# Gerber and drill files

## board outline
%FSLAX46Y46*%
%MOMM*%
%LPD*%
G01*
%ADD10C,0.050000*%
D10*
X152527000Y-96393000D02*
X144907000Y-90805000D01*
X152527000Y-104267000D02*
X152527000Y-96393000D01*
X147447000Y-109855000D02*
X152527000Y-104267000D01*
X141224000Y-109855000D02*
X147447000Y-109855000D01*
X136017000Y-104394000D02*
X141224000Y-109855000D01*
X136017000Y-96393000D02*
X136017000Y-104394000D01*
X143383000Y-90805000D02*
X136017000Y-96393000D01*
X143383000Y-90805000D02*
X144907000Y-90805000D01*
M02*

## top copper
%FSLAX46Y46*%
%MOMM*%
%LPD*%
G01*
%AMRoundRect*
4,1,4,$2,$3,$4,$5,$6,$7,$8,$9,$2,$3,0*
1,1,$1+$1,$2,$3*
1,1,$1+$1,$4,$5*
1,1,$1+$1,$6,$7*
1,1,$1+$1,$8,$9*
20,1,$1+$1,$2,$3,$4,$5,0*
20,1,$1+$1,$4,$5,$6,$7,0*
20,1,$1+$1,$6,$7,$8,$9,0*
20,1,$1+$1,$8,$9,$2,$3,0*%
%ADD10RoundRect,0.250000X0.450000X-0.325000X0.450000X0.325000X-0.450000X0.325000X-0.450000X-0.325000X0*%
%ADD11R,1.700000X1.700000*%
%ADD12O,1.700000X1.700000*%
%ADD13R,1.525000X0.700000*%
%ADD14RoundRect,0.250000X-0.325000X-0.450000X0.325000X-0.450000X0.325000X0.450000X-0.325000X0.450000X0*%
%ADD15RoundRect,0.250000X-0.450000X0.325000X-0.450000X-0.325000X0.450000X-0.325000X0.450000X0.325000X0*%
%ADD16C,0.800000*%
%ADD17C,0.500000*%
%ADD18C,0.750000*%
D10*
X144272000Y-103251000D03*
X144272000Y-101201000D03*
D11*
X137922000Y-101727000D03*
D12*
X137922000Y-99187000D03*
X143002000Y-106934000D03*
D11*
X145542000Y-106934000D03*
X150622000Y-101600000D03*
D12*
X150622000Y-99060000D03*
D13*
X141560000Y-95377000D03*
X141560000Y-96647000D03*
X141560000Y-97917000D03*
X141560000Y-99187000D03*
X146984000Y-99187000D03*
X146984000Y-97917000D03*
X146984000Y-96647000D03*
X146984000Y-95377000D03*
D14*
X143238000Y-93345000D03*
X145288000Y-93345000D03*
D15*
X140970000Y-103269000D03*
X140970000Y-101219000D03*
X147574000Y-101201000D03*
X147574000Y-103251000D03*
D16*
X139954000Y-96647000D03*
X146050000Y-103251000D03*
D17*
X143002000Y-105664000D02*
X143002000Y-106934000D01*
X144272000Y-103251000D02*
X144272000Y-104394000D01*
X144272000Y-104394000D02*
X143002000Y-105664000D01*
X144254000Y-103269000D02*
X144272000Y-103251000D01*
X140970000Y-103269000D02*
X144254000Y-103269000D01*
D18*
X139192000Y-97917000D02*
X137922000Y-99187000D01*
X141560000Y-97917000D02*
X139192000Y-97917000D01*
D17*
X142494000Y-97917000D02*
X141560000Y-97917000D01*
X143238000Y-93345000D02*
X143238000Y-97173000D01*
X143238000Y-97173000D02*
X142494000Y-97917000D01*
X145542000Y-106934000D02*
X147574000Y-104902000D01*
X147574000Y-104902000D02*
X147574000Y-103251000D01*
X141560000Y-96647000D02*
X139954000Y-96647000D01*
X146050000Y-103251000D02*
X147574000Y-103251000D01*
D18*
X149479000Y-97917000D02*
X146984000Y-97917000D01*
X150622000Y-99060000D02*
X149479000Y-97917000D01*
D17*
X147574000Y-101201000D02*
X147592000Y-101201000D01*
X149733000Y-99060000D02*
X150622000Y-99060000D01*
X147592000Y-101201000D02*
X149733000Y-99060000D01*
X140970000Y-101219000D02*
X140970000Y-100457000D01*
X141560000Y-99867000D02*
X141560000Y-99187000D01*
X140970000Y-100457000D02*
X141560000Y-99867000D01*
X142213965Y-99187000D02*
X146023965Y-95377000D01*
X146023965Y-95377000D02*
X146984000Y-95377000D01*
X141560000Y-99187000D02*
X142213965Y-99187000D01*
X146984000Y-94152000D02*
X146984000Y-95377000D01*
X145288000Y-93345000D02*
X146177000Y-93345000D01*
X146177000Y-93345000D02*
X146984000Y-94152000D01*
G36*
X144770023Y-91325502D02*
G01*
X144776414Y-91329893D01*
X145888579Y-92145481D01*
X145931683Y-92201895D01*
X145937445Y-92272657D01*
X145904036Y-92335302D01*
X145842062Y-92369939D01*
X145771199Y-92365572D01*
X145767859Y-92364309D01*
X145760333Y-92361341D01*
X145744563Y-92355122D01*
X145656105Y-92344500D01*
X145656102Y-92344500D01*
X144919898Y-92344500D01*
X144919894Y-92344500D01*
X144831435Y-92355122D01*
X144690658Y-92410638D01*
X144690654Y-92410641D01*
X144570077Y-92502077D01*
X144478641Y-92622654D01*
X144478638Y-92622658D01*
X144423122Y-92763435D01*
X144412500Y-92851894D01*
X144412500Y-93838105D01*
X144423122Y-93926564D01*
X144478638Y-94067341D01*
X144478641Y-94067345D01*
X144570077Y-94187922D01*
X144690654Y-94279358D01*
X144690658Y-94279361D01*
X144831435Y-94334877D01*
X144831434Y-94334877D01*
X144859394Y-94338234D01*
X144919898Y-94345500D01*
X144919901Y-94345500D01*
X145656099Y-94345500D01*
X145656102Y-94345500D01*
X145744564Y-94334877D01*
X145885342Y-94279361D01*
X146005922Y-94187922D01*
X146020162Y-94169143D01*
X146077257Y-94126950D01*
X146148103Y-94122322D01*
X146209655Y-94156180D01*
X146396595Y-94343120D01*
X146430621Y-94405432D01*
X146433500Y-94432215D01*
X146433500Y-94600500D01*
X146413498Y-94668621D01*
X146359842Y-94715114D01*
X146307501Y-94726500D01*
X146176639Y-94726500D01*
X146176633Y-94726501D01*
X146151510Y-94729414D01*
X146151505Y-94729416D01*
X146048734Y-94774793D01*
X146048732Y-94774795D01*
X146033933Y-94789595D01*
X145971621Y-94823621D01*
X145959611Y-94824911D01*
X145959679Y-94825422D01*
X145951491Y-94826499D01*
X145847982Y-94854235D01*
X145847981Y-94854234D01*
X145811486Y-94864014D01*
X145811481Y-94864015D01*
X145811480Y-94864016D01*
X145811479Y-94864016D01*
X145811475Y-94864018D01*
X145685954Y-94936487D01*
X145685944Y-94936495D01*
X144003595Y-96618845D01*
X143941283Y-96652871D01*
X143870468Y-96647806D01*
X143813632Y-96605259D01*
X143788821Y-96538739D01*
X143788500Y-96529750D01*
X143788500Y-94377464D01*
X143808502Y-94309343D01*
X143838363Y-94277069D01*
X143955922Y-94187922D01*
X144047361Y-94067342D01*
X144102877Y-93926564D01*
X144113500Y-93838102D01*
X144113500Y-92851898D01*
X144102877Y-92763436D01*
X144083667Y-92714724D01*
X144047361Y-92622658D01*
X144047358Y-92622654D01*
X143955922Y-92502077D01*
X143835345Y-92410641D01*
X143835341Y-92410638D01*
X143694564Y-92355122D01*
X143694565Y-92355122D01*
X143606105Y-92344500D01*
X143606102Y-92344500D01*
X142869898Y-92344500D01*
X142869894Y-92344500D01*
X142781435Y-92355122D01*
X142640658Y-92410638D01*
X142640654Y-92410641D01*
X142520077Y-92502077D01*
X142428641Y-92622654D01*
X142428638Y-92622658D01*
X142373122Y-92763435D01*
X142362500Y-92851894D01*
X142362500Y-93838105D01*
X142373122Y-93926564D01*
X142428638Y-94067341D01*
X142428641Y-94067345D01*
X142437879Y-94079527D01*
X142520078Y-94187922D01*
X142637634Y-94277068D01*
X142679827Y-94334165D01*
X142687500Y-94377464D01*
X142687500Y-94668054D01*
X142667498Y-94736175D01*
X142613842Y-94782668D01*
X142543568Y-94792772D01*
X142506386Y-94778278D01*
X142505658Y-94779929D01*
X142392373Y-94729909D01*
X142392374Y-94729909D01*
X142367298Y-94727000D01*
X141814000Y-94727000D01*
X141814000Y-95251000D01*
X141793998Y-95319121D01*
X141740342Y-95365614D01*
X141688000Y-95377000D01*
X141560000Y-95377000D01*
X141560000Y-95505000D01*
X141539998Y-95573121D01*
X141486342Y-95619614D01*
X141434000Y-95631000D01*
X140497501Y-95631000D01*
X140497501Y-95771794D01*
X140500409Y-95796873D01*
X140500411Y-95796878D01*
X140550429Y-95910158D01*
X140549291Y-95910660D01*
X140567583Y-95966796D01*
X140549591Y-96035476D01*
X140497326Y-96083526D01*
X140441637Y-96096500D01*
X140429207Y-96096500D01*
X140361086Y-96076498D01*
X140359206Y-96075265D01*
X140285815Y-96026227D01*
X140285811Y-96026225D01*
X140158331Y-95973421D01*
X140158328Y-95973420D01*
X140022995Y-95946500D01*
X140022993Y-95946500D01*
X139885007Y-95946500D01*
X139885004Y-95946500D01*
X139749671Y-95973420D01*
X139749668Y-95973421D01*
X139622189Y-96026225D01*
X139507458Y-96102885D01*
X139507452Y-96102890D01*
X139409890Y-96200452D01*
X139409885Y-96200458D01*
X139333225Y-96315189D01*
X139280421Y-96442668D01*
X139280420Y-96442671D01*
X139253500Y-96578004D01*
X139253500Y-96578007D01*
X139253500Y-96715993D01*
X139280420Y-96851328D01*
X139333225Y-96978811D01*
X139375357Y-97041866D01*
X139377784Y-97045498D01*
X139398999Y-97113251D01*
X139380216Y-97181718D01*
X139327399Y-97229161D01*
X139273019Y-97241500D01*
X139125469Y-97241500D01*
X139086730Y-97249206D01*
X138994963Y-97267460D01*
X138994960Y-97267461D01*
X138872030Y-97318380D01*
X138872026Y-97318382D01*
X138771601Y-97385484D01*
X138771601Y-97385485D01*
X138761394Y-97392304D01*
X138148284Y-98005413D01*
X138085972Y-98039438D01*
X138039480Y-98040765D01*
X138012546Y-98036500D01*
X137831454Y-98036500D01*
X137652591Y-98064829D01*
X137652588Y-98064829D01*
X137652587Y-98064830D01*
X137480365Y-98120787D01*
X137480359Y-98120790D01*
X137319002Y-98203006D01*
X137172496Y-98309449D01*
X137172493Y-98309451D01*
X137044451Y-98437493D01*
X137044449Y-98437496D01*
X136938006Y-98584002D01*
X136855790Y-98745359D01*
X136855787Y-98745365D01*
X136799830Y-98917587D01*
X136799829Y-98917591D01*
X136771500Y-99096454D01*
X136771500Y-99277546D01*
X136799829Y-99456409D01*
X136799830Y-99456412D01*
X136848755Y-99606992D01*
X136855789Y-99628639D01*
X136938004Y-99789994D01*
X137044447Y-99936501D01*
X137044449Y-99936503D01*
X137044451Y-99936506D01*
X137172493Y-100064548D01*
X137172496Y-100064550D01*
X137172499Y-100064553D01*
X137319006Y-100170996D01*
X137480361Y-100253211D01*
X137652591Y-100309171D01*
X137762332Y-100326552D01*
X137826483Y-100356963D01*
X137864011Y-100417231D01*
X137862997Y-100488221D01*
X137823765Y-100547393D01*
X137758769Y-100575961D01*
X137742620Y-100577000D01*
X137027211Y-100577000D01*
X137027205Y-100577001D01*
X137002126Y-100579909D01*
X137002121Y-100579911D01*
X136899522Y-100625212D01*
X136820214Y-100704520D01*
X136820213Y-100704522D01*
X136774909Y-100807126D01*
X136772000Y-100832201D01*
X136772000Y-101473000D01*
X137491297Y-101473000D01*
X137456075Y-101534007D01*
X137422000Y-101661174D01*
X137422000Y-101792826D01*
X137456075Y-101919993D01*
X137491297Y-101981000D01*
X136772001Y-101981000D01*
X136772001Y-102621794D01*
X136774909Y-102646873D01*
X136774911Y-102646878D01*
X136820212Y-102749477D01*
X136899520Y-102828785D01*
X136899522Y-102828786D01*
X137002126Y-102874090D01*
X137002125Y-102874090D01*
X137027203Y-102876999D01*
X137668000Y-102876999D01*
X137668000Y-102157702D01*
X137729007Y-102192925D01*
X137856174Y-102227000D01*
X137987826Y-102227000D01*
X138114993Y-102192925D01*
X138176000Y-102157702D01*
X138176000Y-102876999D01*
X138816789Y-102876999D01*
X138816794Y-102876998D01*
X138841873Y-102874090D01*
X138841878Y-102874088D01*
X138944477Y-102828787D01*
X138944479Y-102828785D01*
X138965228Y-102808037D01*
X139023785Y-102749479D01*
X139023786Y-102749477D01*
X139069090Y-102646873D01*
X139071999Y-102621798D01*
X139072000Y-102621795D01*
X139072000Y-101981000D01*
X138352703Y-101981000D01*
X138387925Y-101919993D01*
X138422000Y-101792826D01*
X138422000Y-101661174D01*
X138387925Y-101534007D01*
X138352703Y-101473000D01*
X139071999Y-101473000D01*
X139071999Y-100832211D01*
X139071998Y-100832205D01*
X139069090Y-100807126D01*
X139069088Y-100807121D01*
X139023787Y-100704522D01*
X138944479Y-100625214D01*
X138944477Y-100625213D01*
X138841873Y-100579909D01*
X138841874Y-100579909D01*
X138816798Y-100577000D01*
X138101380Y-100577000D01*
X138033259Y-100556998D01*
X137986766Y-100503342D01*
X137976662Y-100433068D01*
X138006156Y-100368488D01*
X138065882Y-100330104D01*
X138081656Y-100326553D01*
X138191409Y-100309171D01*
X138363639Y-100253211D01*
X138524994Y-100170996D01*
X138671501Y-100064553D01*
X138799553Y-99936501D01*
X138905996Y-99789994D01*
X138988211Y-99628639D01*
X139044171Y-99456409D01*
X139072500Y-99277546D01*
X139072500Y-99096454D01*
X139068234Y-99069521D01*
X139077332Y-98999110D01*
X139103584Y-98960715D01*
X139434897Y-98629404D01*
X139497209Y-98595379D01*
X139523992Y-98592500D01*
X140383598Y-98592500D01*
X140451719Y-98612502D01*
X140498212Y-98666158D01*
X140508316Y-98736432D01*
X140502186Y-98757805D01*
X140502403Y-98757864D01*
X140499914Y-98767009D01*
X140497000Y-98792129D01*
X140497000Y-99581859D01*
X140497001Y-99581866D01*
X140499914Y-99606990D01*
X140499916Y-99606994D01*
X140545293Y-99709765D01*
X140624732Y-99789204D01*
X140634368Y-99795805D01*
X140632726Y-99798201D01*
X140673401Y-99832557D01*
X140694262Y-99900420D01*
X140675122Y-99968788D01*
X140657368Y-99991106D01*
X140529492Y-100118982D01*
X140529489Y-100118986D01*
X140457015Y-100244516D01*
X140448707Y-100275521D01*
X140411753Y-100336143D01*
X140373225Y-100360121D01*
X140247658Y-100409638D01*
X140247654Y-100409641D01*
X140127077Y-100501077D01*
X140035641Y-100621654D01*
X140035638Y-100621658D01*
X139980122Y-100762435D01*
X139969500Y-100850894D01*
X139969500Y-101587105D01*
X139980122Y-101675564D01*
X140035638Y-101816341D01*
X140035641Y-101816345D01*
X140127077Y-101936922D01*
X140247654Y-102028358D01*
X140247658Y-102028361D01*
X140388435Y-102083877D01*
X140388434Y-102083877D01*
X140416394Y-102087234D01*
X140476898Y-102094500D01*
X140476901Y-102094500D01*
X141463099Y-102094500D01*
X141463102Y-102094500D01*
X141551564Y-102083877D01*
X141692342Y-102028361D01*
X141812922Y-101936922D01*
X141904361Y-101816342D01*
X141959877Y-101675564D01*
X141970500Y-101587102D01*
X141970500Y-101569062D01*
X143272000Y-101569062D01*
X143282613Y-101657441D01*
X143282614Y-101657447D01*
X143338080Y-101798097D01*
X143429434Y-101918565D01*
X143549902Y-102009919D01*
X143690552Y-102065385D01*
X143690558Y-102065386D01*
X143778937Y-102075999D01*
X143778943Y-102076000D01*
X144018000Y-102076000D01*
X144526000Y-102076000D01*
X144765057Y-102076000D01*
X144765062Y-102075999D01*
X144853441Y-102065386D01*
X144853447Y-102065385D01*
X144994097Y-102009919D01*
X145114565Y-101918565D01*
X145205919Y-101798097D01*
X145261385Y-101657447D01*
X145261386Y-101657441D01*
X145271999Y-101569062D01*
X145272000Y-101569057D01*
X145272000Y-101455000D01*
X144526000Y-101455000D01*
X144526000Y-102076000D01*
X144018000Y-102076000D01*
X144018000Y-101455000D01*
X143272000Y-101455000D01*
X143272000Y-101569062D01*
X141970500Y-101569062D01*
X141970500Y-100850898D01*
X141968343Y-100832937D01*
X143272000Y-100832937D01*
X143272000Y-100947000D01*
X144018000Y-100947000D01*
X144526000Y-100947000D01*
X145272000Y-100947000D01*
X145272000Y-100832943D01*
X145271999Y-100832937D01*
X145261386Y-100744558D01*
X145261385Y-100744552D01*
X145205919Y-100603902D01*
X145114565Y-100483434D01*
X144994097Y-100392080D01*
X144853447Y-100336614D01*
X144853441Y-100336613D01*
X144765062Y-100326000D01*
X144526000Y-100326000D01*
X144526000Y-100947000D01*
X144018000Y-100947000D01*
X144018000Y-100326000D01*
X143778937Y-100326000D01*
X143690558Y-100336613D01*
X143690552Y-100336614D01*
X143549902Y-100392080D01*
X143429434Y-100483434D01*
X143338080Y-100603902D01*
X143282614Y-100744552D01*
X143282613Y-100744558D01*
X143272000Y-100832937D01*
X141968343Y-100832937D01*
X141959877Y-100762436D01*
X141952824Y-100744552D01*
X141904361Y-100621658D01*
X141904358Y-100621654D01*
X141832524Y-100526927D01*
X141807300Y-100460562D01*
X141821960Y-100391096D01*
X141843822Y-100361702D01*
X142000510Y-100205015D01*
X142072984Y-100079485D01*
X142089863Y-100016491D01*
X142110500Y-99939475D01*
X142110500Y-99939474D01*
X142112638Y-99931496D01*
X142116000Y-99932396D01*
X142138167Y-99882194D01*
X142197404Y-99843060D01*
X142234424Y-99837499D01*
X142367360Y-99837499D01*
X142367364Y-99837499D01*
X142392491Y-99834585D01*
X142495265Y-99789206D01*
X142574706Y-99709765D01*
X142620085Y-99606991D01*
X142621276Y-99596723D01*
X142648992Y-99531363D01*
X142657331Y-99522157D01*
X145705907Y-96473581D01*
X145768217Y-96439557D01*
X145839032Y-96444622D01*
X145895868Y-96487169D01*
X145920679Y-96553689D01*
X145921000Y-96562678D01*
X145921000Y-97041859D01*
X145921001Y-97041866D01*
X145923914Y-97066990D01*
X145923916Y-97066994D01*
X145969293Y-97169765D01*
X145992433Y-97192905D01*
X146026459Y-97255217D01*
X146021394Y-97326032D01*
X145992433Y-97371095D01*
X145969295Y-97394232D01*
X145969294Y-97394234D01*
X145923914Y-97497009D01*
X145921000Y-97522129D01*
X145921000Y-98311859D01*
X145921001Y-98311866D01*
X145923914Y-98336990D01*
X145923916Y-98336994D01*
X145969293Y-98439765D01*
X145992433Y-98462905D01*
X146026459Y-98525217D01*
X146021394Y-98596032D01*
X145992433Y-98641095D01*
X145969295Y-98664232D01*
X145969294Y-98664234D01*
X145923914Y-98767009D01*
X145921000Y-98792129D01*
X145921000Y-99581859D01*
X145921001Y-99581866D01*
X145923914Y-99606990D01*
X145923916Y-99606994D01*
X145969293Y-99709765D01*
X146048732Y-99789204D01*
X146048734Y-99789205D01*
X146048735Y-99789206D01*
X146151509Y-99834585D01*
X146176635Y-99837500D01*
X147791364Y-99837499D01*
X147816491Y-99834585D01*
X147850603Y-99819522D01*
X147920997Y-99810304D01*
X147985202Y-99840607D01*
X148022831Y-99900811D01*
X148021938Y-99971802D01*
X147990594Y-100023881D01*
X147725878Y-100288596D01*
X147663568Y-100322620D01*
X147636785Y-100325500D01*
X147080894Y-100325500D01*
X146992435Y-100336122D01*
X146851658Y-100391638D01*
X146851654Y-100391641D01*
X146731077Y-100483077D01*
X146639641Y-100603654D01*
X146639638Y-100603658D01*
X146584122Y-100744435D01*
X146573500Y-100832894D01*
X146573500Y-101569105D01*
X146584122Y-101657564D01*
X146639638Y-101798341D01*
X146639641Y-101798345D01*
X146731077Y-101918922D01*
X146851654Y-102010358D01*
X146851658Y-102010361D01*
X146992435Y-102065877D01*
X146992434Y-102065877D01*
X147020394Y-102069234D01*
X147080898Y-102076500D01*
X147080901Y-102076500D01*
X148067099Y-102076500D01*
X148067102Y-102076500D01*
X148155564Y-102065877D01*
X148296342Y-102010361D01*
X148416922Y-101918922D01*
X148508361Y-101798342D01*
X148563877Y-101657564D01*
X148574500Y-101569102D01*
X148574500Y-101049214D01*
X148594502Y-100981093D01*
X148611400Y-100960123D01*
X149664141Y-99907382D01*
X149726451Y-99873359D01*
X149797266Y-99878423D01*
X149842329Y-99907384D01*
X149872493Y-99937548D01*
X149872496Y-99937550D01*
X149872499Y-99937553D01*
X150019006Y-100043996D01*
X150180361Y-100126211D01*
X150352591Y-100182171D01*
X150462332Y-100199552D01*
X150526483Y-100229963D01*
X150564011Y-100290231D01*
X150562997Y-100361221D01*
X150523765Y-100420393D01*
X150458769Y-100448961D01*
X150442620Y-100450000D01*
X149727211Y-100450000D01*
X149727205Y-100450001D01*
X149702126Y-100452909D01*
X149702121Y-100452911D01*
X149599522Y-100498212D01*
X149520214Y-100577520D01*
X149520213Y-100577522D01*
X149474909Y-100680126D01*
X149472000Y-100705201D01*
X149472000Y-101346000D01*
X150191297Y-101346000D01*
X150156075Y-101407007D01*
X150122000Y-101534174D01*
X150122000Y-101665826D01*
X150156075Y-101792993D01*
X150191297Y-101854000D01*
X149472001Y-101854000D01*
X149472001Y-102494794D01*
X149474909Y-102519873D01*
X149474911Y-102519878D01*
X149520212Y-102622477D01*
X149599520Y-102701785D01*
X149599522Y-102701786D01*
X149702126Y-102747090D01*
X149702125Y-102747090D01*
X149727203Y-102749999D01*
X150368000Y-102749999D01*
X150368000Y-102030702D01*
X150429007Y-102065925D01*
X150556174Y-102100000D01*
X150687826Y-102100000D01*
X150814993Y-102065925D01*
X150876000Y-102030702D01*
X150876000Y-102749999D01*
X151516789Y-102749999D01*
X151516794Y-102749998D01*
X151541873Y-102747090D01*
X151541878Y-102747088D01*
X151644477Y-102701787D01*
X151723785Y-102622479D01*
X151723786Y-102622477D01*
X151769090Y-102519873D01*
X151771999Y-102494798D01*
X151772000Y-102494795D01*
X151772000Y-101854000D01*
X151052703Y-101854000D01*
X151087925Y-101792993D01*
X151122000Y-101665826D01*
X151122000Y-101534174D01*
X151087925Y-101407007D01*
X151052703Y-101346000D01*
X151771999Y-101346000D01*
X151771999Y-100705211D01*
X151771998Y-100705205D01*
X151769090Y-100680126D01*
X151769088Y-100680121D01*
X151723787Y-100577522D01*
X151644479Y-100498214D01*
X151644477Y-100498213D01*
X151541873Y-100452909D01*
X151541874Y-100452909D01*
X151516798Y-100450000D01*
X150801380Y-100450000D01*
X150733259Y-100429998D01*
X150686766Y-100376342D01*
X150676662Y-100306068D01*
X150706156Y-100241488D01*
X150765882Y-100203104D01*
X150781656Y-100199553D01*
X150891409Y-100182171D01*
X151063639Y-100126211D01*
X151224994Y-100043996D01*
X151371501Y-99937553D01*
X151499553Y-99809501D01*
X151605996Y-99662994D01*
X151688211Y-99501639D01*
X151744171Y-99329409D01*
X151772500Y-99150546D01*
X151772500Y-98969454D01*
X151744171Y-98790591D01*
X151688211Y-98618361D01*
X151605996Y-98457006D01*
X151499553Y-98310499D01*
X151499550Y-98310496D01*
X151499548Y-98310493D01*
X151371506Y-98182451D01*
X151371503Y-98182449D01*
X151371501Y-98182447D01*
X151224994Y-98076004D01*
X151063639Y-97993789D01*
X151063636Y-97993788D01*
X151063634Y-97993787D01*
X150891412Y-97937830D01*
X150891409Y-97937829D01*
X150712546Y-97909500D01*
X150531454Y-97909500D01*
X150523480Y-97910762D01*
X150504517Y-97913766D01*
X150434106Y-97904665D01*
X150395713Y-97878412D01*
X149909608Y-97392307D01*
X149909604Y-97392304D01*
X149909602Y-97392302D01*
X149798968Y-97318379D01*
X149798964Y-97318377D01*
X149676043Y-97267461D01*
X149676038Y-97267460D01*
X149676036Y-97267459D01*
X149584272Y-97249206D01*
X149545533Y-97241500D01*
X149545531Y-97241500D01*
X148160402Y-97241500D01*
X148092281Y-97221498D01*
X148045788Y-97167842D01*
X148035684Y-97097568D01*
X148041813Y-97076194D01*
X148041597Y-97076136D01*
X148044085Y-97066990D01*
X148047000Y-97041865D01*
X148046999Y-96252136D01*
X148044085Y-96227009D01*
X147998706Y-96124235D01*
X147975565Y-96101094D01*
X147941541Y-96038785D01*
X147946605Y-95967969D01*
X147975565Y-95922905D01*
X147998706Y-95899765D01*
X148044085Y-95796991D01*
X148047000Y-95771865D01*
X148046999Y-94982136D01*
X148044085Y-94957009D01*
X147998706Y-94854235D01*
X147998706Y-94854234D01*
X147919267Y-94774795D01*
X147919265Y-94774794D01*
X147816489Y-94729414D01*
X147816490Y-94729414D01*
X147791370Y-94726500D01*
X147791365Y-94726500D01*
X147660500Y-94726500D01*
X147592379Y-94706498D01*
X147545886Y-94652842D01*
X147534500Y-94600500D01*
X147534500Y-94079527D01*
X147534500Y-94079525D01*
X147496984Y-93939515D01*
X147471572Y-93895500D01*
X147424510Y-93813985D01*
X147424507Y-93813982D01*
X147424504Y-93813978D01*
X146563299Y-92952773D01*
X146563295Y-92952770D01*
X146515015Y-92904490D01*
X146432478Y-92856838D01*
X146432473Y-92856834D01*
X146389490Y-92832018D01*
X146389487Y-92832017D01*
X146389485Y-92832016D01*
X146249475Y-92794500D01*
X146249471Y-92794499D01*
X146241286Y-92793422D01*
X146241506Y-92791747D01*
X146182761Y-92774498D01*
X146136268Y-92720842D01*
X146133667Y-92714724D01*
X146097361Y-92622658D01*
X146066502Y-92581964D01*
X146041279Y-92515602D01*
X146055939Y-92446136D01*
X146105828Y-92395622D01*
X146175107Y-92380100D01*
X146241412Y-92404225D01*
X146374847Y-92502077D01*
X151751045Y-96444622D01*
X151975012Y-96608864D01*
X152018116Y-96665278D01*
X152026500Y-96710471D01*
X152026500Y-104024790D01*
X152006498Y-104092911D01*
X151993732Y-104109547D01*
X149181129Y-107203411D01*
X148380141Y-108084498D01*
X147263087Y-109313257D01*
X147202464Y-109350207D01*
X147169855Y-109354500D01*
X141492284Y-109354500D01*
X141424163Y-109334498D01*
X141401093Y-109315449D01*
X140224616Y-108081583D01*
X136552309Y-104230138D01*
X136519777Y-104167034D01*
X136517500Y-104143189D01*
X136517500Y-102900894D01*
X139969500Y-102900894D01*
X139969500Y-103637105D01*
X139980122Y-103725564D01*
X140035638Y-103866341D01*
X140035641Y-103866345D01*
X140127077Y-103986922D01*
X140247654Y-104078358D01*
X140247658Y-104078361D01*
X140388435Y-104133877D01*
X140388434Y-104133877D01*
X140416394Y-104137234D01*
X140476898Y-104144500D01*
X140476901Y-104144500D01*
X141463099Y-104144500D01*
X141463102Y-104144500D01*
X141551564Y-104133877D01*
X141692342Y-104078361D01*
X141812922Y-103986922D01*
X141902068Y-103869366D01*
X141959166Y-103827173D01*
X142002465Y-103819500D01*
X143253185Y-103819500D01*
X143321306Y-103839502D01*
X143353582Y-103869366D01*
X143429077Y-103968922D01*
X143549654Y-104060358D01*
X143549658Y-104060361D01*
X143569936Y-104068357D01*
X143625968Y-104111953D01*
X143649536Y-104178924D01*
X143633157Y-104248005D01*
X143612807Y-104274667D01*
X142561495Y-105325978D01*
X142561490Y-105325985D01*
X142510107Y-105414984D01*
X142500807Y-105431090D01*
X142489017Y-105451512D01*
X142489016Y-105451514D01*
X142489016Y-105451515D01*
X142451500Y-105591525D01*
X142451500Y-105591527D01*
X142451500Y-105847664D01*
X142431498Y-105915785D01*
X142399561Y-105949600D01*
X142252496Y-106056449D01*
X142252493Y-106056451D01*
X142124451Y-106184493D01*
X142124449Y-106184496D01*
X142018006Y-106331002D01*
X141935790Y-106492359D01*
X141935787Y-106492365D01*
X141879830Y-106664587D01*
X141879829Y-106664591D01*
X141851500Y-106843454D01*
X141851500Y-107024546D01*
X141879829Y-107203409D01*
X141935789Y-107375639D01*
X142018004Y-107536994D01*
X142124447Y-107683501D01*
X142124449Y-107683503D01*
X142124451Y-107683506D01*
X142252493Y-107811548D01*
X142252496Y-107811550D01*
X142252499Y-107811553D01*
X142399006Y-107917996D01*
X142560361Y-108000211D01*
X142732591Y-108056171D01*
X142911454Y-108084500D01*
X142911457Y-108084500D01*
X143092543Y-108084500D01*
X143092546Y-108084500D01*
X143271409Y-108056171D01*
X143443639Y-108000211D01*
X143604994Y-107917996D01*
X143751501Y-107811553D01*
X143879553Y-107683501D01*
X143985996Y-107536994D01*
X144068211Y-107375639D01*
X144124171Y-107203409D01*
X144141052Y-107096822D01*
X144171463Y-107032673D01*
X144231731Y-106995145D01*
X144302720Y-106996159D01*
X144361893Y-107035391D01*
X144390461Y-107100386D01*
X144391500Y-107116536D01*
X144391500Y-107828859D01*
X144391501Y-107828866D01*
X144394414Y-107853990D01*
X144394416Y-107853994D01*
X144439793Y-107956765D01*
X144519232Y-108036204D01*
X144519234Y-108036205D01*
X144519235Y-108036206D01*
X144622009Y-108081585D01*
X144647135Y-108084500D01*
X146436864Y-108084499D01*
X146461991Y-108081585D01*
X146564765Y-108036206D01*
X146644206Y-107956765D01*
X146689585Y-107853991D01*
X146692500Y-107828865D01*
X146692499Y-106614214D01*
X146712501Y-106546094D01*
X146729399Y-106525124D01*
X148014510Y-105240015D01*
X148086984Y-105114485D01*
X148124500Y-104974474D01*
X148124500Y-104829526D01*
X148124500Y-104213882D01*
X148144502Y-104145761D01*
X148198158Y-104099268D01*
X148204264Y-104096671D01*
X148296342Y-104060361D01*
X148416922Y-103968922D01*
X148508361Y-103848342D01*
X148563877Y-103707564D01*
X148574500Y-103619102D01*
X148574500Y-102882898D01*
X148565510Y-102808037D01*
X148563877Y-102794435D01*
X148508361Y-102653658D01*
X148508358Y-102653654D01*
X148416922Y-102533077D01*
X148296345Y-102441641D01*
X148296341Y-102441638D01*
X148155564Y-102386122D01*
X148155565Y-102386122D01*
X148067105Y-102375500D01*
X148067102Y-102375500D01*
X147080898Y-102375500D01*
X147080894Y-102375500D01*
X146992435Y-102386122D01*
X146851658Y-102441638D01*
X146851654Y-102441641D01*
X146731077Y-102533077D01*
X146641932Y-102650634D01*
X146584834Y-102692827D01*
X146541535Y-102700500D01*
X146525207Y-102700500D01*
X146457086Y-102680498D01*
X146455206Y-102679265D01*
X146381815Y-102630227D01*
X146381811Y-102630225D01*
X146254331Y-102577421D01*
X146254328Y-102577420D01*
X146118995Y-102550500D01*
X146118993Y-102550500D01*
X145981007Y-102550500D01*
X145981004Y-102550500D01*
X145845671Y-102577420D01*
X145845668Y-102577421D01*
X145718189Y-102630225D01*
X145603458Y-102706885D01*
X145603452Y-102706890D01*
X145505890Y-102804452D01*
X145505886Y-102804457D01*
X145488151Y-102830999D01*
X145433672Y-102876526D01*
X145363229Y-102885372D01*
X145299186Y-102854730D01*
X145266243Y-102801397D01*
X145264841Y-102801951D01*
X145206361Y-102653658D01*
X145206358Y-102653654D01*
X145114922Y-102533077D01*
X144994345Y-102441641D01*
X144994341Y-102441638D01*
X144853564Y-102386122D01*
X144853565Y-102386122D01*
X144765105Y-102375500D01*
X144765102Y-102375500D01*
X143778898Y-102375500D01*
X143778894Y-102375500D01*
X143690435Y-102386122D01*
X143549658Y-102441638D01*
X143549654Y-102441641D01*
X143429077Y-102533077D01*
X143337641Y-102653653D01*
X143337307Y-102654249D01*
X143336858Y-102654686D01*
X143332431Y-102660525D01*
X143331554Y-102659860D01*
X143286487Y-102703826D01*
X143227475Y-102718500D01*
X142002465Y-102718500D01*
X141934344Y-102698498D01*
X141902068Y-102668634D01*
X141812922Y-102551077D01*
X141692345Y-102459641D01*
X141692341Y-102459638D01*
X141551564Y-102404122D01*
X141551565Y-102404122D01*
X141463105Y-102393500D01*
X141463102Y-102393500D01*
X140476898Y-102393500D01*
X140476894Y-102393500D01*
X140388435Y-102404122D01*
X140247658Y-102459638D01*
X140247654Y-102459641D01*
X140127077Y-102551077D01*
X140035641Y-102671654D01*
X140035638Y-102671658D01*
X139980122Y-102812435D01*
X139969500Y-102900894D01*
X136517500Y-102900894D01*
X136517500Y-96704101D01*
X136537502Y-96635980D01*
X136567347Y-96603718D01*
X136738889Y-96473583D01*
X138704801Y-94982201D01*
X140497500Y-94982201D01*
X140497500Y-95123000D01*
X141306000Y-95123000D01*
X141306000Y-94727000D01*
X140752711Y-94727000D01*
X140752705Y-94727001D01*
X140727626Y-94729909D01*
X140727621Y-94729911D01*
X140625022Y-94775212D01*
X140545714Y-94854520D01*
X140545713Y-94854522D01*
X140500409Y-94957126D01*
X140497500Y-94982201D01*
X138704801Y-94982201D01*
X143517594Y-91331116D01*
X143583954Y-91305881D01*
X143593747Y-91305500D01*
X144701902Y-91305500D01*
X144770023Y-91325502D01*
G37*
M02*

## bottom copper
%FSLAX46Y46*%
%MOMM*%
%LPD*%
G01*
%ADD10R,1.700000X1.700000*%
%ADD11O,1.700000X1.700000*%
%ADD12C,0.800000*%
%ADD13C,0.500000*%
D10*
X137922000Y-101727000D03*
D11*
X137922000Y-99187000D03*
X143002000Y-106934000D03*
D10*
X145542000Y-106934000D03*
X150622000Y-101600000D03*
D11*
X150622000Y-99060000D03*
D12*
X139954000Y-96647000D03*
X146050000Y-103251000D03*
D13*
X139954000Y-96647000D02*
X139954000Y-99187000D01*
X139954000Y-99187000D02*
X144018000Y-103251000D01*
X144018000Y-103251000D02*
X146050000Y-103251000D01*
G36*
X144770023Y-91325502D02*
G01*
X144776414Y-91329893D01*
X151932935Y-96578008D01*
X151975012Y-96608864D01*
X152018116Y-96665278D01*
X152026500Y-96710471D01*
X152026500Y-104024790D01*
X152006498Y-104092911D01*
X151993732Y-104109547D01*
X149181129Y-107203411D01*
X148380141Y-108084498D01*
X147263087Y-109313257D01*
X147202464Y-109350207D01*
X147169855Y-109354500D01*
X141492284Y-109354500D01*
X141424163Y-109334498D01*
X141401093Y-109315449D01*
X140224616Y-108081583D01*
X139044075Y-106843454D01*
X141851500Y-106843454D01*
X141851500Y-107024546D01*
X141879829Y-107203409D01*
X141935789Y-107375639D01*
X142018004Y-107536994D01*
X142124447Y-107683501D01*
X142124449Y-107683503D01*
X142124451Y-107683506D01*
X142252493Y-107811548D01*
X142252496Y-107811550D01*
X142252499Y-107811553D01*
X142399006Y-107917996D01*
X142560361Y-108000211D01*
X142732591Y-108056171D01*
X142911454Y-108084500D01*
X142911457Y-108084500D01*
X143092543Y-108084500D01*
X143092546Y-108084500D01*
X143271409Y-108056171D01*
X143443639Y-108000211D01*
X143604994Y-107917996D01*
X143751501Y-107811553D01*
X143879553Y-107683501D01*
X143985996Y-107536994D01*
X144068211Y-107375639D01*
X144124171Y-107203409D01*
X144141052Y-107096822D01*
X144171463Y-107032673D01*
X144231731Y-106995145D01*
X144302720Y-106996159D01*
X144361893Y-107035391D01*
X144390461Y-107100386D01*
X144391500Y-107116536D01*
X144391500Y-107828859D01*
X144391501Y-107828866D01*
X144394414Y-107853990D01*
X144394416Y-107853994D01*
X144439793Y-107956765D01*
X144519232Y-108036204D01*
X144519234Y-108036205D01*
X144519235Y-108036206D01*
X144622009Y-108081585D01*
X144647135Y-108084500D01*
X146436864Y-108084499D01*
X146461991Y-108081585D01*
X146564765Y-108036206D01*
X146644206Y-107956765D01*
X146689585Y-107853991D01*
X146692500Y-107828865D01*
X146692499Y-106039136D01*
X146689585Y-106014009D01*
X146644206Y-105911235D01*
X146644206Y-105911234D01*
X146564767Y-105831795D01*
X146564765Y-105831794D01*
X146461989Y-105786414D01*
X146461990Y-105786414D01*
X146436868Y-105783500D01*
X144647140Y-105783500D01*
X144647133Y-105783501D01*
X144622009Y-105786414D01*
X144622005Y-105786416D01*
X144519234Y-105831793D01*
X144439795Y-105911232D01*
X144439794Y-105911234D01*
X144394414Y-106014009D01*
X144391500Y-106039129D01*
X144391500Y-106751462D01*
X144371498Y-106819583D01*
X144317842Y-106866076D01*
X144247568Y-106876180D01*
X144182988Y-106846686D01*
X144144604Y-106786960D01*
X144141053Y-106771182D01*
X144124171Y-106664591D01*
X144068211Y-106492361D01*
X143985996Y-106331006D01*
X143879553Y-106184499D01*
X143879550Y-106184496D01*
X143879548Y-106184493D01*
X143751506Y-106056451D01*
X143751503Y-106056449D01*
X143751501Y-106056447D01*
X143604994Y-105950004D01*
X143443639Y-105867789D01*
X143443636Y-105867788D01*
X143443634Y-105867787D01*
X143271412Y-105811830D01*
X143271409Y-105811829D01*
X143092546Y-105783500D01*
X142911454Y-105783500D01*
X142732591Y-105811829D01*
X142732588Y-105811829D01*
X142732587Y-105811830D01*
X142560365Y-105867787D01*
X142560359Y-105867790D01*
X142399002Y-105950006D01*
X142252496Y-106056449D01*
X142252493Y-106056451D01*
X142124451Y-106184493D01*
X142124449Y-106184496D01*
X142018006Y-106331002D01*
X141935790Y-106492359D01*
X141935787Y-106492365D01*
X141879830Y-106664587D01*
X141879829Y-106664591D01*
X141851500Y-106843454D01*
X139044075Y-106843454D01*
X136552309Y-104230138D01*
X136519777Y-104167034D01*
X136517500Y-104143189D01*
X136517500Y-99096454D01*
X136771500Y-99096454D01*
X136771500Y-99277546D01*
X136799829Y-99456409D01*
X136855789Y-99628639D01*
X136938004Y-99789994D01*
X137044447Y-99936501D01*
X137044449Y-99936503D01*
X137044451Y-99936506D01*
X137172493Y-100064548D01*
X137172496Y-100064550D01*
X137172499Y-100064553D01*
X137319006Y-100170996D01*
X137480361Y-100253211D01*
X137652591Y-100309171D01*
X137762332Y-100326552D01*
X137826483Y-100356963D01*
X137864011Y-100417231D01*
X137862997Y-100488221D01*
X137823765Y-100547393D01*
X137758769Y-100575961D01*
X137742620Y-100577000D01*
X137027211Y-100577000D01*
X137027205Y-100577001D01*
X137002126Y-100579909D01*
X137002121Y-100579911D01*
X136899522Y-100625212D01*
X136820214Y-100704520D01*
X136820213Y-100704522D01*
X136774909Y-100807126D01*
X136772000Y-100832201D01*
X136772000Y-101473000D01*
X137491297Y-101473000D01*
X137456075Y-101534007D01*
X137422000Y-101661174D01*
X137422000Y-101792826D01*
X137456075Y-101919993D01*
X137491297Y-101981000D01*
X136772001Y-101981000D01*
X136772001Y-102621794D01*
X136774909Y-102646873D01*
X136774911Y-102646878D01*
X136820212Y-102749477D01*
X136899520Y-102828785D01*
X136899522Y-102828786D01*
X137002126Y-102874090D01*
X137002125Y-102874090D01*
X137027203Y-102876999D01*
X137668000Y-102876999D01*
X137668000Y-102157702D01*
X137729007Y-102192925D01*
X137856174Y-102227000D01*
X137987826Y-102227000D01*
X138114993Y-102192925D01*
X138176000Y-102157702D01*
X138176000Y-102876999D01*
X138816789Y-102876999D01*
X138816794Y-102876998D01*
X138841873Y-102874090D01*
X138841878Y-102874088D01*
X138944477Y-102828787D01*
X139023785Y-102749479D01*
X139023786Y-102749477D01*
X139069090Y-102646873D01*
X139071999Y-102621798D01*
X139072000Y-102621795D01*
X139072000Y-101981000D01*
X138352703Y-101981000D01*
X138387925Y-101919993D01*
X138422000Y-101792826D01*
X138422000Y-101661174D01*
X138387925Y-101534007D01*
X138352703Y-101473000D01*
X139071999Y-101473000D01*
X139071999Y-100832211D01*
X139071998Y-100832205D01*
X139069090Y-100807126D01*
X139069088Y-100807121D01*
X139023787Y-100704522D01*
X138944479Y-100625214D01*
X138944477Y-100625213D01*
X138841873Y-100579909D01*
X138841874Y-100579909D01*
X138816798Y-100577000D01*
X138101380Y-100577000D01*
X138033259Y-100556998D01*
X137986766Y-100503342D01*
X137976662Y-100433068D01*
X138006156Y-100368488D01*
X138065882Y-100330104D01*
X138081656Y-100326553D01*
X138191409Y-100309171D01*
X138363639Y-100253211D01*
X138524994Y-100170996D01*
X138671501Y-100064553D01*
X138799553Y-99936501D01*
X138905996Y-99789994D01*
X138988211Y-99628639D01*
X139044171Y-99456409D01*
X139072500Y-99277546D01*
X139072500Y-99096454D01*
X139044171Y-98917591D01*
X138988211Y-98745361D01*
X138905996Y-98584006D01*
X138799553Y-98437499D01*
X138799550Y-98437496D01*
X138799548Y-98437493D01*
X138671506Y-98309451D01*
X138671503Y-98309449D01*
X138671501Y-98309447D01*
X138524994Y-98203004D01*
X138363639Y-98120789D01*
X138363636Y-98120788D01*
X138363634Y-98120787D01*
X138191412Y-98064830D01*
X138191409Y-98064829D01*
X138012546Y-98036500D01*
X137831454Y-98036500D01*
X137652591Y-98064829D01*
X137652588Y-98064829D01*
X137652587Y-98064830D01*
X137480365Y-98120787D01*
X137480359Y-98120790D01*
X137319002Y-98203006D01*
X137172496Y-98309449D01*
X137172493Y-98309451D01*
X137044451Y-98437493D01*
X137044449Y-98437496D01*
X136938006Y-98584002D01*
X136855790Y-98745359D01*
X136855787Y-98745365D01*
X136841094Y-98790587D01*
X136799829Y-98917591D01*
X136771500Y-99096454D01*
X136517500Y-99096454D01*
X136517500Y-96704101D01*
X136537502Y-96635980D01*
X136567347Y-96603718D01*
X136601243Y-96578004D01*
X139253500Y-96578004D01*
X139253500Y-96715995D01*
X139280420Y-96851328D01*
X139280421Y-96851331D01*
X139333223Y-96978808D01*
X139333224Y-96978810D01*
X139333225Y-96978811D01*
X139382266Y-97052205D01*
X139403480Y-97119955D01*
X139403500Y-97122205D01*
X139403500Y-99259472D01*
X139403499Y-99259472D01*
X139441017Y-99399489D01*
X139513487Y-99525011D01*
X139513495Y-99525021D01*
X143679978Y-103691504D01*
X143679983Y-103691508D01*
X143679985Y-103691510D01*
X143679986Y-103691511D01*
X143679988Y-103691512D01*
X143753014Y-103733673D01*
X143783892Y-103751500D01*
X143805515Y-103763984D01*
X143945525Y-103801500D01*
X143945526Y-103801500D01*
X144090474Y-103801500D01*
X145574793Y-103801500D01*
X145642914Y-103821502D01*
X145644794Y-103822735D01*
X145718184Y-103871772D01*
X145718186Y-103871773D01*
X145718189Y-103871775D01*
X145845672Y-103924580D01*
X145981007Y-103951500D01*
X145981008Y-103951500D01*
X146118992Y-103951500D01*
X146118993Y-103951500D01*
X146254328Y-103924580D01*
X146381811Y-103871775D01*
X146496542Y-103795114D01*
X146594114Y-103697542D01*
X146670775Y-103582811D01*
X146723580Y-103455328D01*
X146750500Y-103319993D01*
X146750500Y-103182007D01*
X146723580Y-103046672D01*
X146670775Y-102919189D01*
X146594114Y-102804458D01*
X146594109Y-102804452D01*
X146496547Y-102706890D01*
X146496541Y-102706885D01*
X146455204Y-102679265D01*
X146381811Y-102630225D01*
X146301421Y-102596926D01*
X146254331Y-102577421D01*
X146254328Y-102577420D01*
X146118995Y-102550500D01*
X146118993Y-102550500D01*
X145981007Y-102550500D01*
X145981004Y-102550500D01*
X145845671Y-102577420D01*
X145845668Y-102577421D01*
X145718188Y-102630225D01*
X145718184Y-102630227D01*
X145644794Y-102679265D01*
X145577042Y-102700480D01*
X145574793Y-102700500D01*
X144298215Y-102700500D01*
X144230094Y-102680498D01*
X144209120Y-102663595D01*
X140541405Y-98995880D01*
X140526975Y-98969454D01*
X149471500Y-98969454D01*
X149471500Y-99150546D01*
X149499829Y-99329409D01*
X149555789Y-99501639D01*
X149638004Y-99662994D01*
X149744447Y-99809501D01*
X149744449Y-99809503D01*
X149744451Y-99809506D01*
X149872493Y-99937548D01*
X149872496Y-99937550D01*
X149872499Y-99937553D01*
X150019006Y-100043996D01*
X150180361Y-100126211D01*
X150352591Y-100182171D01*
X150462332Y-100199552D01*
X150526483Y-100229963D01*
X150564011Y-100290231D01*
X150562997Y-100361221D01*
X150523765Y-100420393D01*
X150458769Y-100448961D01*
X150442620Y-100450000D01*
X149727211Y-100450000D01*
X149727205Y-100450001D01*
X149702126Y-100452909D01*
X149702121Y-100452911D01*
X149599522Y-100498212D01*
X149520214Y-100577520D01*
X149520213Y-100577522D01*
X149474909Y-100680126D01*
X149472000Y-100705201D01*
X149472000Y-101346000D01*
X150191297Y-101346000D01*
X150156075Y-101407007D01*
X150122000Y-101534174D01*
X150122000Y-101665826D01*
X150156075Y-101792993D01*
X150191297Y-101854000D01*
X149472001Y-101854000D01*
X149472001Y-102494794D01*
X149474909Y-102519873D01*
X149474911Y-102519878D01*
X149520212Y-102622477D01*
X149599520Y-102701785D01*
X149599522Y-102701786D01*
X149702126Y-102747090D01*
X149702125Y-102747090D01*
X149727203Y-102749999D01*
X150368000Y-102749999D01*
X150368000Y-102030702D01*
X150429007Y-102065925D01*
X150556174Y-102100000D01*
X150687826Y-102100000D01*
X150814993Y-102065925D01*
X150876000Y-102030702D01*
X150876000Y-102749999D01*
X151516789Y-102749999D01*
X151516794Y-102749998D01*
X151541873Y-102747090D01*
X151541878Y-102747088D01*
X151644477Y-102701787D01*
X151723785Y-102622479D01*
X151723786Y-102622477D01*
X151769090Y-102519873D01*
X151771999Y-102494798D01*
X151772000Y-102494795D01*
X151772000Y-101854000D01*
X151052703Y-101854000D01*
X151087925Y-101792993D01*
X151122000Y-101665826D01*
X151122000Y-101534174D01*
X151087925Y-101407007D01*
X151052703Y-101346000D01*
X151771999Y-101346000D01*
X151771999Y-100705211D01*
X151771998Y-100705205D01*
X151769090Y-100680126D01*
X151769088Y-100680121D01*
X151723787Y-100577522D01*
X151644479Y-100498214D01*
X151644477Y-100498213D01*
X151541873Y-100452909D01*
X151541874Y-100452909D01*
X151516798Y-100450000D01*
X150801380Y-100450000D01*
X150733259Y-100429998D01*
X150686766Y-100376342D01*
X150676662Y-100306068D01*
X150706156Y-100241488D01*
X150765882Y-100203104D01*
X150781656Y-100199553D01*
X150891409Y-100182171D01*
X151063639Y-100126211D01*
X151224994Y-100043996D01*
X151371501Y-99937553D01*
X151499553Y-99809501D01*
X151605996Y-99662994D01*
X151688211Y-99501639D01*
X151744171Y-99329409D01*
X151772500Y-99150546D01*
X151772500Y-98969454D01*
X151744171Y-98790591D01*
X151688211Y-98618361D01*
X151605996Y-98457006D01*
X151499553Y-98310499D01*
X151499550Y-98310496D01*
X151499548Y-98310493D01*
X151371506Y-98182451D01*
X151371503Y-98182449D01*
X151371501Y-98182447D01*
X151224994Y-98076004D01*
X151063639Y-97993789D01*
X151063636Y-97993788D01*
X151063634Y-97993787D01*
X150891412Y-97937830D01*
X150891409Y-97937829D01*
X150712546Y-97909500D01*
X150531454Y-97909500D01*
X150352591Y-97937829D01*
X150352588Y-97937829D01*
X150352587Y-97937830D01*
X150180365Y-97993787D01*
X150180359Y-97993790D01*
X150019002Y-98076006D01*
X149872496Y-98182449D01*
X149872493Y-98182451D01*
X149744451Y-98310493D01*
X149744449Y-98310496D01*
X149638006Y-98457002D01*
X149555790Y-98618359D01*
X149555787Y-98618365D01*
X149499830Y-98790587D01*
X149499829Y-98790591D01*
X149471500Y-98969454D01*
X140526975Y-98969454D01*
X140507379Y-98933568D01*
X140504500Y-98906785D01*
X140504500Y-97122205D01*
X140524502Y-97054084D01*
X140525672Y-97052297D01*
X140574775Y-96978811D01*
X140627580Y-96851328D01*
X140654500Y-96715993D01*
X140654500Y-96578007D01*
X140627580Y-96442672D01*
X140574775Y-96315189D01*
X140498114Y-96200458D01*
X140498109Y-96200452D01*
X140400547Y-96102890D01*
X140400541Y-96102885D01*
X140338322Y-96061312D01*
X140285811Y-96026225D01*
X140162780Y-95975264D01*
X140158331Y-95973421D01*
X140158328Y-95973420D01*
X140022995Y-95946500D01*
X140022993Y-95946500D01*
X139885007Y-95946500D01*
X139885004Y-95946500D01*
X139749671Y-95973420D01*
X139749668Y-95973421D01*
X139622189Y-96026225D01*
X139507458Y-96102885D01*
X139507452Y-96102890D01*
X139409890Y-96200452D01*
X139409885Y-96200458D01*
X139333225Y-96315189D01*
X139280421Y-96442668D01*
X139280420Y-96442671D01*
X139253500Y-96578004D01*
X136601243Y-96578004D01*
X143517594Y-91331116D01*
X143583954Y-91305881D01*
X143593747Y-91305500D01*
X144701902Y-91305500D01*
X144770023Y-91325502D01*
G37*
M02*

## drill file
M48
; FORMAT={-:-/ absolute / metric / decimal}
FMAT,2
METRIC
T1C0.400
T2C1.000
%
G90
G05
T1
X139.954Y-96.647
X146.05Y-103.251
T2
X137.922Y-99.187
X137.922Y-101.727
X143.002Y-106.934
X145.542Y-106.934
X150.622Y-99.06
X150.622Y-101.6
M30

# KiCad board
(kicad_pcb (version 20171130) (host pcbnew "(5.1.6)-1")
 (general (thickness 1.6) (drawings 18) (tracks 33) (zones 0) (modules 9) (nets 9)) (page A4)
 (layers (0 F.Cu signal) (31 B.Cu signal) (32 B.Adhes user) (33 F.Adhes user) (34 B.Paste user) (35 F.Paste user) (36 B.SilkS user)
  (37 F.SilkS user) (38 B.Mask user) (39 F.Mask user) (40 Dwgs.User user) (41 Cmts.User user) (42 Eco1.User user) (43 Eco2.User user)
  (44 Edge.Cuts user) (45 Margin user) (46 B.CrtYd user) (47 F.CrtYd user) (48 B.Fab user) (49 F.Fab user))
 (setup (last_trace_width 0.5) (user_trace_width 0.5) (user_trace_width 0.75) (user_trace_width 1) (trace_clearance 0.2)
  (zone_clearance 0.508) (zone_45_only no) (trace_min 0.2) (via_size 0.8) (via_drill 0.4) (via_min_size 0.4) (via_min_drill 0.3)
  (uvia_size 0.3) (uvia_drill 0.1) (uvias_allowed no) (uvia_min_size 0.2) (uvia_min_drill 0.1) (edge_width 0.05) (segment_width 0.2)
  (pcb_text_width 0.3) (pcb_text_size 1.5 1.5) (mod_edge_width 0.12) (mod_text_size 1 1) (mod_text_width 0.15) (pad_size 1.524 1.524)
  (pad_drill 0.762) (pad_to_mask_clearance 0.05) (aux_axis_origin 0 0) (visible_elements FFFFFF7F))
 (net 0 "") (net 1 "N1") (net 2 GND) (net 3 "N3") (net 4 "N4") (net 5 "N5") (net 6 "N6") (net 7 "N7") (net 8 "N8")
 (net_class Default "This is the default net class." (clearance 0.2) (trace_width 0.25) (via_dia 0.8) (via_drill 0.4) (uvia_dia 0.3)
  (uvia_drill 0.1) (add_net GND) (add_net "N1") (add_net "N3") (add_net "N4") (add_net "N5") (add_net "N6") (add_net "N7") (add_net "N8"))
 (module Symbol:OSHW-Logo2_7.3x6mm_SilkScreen (layer B.Cu) (at 144.145 94.234 180)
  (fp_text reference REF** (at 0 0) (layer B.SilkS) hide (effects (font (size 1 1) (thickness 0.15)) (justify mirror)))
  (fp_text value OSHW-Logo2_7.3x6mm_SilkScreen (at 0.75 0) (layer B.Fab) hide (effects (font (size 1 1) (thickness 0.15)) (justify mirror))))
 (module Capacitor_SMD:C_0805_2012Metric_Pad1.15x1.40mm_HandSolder (layer F.Cu) (at 144.272 102.226 90)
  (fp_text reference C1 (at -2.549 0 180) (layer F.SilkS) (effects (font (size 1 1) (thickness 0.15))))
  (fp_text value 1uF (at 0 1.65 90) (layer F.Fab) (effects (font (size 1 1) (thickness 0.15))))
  (pad 1 smd roundrect (at -1.025 0 90) (size 1.15 1.4) (layers F.Cu F.Paste F.Mask) (roundrect_rratio 0.217391) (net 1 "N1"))
  (pad 2 smd roundrect (at 1.025 0 90) (size 1.15 1.4) (layers F.Cu F.Paste F.Mask) (roundrect_rratio 0.217391) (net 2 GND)))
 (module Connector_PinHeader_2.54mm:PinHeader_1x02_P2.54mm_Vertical (layer F.Cu) (at 137.922 101.727 180)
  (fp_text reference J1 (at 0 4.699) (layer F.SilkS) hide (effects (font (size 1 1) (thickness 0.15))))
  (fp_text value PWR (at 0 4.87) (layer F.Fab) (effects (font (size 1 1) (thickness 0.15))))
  (pad 1 thru_hole rect (at 0 0 180) (size 1.7 1.7) (drill 1) (layers *.Cu *.Mask) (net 2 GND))
  (pad 2 thru_hole oval (at 0 2.54 180) (size 1.7 1.7) (drill 1) (layers *.Cu *.Mask) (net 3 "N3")))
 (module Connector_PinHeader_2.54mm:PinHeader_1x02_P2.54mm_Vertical (layer F.Cu) (at 145.542 106.934 270)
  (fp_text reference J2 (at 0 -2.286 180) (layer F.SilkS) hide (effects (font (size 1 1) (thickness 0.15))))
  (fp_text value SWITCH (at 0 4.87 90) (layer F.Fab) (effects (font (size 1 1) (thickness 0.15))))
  (pad 2 thru_hole oval (at 0 2.54 270) (size 1.7 1.7) (drill 1) (layers *.Cu *.Mask) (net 1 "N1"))
  (pad 1 thru_hole rect (at 0 0 270) (size 1.7 1.7) (drill 1) (layers *.Cu *.Mask) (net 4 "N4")))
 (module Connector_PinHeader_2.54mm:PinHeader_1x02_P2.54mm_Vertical (layer F.Cu) (at 150.622 101.6 180)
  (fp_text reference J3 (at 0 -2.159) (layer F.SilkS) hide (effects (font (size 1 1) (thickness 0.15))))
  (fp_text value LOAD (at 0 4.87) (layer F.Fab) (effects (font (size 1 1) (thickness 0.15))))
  (pad 1 thru_hole rect (at 0 0 180) (size 1.7 1.7) (drill 1) (layers *.Cu *.Mask) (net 2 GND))
  (pad 2 thru_hole oval (at 0 2.54 180) (size 1.7 1.7) (drill 1) (layers *.Cu *.Mask) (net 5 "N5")))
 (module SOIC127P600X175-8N (layer F.Cu) (at 144.272 97.282)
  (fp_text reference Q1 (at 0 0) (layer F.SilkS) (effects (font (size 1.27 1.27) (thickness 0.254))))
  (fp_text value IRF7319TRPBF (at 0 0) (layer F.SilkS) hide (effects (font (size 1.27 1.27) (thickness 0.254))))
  (pad 1 smd rect (at -2.712 -1.905 90) (size 0.7 1.525) (layers F.Cu F.Paste F.Mask) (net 2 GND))
  (pad 2 smd rect (at -2.712 -0.635 90) (size 0.7 1.525) (layers F.Cu F.Paste F.Mask) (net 4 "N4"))
  (pad 3 smd rect (at -2.712 0.635 90) (size 0.7 1.525) (layers F.Cu F.Paste F.Mask) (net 3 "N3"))
  (pad 4 smd rect (at -2.712 1.905 90) (size 0.7 1.525) (layers F.Cu F.Paste F.Mask) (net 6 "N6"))
  (pad 5 smd rect (at 2.712 1.905 90) (size 0.7 1.525) (layers F.Cu F.Paste F.Mask) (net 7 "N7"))
  (pad 6 smd rect (at 2.712 0.635 90) (size 0.7 1.525) (layers F.Cu F.Paste F.Mask) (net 5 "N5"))
  (pad 7 smd rect (at 2.712 -0.635 90) (size 0.7 1.525) (layers F.Cu F.Paste F.Mask) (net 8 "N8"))
  (pad 8 smd rect (at 2.712 -1.905 90) (size 0.7 1.525) (layers F.Cu F.Paste F.Mask) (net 6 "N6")))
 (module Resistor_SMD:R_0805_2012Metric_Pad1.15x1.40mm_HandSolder (layer F.Cu) (at 144.263 93.345)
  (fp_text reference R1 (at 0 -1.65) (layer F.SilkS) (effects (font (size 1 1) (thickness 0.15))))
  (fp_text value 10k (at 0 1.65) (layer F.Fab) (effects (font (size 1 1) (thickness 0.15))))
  (pad 1 smd roundrect (at -1.025 0) (size 1.15 1.4) (layers F.Cu F.Paste F.Mask) (roundrect_rratio 0.217391) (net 3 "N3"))
  (pad 2 smd roundrect (at 1.025 0) (size 1.15 1.4) (layers F.Cu F.Paste F.Mask) (roundrect_rratio 0.217391) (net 6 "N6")))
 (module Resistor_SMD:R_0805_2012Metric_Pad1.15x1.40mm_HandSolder (layer F.Cu) (at 140.97 102.244 270)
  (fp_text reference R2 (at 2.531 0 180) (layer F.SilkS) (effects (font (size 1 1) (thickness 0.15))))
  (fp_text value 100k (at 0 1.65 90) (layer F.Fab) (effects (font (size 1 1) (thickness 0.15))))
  (pad 2 smd roundrect (at 1.025 0 270) (size 1.15 1.4) (layers F.Cu F.Paste F.Mask) (roundrect_rratio 0.217391) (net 1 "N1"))
  (pad 1 smd roundrect (at -1.025 0 270) (size 1.15 1.4) (layers F.Cu F.Paste F.Mask) (roundrect_rratio 0.217391) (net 6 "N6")))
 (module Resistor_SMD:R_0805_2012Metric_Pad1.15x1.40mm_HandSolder (layer F.Cu) (at 147.574 102.226 270)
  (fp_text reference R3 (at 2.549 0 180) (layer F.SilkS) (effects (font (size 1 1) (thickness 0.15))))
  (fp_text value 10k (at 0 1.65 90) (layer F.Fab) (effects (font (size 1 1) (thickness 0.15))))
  (pad 1 smd roundrect (at -1.025 0 270) (size 1.15 1.4) (layers F.Cu F.Paste F.Mask) (roundrect_rratio 0.217391) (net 5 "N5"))
  (pad 2 smd roundrect (at 1.025 0 270) (size 1.15 1.4) (layers F.Cu F.Paste F.Mask) (roundrect_rratio 0.217391) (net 4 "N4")))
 (gr_line (start 152.527 96.393) (end 144.907 90.805) (layer Edge.Cuts) (width 0.05))
 (gr_line (start 152.527 104.267) (end 152.527 96.393) (layer Edge.Cuts) (width 0.05))
 (gr_line (start 147.447 109.855) (end 152.527 104.267) (layer Edge.Cuts) (width 0.05))
 (gr_line (start 141.224 109.855) (end 147.447 109.855) (layer Edge.Cuts) (width 0.05))
 (gr_line (start 136.017 104.394) (end 141.224 109.855) (layer Edge.Cuts) (width 0.05))
 (gr_line (start 136.017 96.393) (end 136.017 104.394) (layer Edge.Cuts) (width 0.05))
 (gr_line (start 143.383 90.805) (end 136.017 96.393) (layer Edge.Cuts) (width 0.05))
 (gr_line (start 143.383 90.805) (end 144.907 90.805) (layer Edge.Cuts) (width 0.05))
 (segment (start 143.002 105.664) (end 143.002 106.934) (width 0.5) (layer F.Cu) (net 1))
 (segment (start 144.272 103.251) (end 144.272 104.394) (width 0.5) (layer F.Cu) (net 1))
 (segment (start 144.272 104.394) (end 143.002 105.664) (width 0.5) (layer F.Cu) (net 1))
 (segment (start 144.254 103.269) (end 144.272 103.251) (width 0.5) (layer F.Cu) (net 1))
 (segment (start 140.97 103.269) (end 144.254 103.269) (width 0.5) (layer F.Cu) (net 1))
 (segment (start 139.192 97.917) (end 137.922 99.187) (width 0.75) (layer F.Cu) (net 3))
 (segment (start 141.56 97.917) (end 139.192 97.917) (width 0.75) (layer F.Cu) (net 3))
 (segment (start 142.494 97.917) (end 141.56 97.917) (width 0.5) (layer F.Cu) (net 3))
 (segment (start 143.238 93.345) (end 143.238 97.173) (width 0.5) (layer F.Cu) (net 3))
 (segment (start 143.238 97.173) (end 142.494 97.917) (width 0.5) (layer F.Cu) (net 3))
 (segment (start 145.542 106.934) (end 147.574 104.902) (width 0.5) (layer F.Cu) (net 4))
 (segment (start 147.574 104.902) (end 147.574 103.251) (width 0.5) (layer F.Cu) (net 4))
 (via (at 139.954 96.647) (size 0.8) (drill 0.4) (layers F.Cu B.Cu) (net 4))
 (segment (start 141.56 96.647) (end 139.954 96.647) (width 0.5) (layer F.Cu) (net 4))
 (segment (start 139.954 96.647) (end 139.954 99.187) (width 0.5) (layer B.Cu) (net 4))
 (segment (start 139.954 99.187) (end 144.018 103.251) (width 0.5) (layer B.Cu) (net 4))
 (via (at 146.05 103.251) (size 0.8) (drill 0.4) (layers F.Cu B.Cu) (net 4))
 (segment (start 144.018 103.251) (end 146.05 103.251) (width 0.5) (layer B.Cu) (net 4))
 (segment (start 146.05 103.251) (end 147.574 103.251) (width 0.5) (layer F.Cu) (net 4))
 (segment (start 149.479 97.917) (end 146.984 97.917) (width 0.75) (layer F.Cu) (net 5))
 (segment (start 150.622 99.06) (end 149.479 97.917) (width 0.75) (layer F.Cu) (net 5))
 (segment (start 147.574 101.201) (end 147.592 101.201) (width 0.5) (layer F.Cu) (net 5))
 (segment (start 149.733 99.06) (end 150.622 99.06) (width 0.5) (layer F.Cu) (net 5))
 (segment (start 147.592 101.201) (end 149.733 99.06) (width 0.5) (layer F.Cu) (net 5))
 (segment (start 140.97 101.219) (end 140.97 100.457) (width 0.5) (layer F.Cu) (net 6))
 (segment (start 141.56 99.867) (end 141.56 99.187) (width 0.5) (layer F.Cu) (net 6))
 (segment (start 140.97 100.457) (end 141.56 99.867) (width 0.5) (layer F.Cu) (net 6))
 (segment (start 142.213965 99.187) (end 146.023965 95.377) (width 0.5) (layer F.Cu) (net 6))
 (segment (start 146.023965 95.377) (end 146.984 95.377) (width 0.5) (layer F.Cu) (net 6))
 (segment (start 141.56 99.187) (end 142.213965 99.187) (width 0.5) (layer F.Cu) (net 6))
 (segment (start 146.984 94.152) (end 146.984 95.377) (width 0.5) (layer F.Cu) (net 6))
 (segment (start 145.288 93.345) (end 146.177 93.345) (width 0.5) (layer F.Cu) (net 6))
 (segment (start 146.177 93.345) (end 146.984 94.152) (width 0.5) (layer F.Cu) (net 6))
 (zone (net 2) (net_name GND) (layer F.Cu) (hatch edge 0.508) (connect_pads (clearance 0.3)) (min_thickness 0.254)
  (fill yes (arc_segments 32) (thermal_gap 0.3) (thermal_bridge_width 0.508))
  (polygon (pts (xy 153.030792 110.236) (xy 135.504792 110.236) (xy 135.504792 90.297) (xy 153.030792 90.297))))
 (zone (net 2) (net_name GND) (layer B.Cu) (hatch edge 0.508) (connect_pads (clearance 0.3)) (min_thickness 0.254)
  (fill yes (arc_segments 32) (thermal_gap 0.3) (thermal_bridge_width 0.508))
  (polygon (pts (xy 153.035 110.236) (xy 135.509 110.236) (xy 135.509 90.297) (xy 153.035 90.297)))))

